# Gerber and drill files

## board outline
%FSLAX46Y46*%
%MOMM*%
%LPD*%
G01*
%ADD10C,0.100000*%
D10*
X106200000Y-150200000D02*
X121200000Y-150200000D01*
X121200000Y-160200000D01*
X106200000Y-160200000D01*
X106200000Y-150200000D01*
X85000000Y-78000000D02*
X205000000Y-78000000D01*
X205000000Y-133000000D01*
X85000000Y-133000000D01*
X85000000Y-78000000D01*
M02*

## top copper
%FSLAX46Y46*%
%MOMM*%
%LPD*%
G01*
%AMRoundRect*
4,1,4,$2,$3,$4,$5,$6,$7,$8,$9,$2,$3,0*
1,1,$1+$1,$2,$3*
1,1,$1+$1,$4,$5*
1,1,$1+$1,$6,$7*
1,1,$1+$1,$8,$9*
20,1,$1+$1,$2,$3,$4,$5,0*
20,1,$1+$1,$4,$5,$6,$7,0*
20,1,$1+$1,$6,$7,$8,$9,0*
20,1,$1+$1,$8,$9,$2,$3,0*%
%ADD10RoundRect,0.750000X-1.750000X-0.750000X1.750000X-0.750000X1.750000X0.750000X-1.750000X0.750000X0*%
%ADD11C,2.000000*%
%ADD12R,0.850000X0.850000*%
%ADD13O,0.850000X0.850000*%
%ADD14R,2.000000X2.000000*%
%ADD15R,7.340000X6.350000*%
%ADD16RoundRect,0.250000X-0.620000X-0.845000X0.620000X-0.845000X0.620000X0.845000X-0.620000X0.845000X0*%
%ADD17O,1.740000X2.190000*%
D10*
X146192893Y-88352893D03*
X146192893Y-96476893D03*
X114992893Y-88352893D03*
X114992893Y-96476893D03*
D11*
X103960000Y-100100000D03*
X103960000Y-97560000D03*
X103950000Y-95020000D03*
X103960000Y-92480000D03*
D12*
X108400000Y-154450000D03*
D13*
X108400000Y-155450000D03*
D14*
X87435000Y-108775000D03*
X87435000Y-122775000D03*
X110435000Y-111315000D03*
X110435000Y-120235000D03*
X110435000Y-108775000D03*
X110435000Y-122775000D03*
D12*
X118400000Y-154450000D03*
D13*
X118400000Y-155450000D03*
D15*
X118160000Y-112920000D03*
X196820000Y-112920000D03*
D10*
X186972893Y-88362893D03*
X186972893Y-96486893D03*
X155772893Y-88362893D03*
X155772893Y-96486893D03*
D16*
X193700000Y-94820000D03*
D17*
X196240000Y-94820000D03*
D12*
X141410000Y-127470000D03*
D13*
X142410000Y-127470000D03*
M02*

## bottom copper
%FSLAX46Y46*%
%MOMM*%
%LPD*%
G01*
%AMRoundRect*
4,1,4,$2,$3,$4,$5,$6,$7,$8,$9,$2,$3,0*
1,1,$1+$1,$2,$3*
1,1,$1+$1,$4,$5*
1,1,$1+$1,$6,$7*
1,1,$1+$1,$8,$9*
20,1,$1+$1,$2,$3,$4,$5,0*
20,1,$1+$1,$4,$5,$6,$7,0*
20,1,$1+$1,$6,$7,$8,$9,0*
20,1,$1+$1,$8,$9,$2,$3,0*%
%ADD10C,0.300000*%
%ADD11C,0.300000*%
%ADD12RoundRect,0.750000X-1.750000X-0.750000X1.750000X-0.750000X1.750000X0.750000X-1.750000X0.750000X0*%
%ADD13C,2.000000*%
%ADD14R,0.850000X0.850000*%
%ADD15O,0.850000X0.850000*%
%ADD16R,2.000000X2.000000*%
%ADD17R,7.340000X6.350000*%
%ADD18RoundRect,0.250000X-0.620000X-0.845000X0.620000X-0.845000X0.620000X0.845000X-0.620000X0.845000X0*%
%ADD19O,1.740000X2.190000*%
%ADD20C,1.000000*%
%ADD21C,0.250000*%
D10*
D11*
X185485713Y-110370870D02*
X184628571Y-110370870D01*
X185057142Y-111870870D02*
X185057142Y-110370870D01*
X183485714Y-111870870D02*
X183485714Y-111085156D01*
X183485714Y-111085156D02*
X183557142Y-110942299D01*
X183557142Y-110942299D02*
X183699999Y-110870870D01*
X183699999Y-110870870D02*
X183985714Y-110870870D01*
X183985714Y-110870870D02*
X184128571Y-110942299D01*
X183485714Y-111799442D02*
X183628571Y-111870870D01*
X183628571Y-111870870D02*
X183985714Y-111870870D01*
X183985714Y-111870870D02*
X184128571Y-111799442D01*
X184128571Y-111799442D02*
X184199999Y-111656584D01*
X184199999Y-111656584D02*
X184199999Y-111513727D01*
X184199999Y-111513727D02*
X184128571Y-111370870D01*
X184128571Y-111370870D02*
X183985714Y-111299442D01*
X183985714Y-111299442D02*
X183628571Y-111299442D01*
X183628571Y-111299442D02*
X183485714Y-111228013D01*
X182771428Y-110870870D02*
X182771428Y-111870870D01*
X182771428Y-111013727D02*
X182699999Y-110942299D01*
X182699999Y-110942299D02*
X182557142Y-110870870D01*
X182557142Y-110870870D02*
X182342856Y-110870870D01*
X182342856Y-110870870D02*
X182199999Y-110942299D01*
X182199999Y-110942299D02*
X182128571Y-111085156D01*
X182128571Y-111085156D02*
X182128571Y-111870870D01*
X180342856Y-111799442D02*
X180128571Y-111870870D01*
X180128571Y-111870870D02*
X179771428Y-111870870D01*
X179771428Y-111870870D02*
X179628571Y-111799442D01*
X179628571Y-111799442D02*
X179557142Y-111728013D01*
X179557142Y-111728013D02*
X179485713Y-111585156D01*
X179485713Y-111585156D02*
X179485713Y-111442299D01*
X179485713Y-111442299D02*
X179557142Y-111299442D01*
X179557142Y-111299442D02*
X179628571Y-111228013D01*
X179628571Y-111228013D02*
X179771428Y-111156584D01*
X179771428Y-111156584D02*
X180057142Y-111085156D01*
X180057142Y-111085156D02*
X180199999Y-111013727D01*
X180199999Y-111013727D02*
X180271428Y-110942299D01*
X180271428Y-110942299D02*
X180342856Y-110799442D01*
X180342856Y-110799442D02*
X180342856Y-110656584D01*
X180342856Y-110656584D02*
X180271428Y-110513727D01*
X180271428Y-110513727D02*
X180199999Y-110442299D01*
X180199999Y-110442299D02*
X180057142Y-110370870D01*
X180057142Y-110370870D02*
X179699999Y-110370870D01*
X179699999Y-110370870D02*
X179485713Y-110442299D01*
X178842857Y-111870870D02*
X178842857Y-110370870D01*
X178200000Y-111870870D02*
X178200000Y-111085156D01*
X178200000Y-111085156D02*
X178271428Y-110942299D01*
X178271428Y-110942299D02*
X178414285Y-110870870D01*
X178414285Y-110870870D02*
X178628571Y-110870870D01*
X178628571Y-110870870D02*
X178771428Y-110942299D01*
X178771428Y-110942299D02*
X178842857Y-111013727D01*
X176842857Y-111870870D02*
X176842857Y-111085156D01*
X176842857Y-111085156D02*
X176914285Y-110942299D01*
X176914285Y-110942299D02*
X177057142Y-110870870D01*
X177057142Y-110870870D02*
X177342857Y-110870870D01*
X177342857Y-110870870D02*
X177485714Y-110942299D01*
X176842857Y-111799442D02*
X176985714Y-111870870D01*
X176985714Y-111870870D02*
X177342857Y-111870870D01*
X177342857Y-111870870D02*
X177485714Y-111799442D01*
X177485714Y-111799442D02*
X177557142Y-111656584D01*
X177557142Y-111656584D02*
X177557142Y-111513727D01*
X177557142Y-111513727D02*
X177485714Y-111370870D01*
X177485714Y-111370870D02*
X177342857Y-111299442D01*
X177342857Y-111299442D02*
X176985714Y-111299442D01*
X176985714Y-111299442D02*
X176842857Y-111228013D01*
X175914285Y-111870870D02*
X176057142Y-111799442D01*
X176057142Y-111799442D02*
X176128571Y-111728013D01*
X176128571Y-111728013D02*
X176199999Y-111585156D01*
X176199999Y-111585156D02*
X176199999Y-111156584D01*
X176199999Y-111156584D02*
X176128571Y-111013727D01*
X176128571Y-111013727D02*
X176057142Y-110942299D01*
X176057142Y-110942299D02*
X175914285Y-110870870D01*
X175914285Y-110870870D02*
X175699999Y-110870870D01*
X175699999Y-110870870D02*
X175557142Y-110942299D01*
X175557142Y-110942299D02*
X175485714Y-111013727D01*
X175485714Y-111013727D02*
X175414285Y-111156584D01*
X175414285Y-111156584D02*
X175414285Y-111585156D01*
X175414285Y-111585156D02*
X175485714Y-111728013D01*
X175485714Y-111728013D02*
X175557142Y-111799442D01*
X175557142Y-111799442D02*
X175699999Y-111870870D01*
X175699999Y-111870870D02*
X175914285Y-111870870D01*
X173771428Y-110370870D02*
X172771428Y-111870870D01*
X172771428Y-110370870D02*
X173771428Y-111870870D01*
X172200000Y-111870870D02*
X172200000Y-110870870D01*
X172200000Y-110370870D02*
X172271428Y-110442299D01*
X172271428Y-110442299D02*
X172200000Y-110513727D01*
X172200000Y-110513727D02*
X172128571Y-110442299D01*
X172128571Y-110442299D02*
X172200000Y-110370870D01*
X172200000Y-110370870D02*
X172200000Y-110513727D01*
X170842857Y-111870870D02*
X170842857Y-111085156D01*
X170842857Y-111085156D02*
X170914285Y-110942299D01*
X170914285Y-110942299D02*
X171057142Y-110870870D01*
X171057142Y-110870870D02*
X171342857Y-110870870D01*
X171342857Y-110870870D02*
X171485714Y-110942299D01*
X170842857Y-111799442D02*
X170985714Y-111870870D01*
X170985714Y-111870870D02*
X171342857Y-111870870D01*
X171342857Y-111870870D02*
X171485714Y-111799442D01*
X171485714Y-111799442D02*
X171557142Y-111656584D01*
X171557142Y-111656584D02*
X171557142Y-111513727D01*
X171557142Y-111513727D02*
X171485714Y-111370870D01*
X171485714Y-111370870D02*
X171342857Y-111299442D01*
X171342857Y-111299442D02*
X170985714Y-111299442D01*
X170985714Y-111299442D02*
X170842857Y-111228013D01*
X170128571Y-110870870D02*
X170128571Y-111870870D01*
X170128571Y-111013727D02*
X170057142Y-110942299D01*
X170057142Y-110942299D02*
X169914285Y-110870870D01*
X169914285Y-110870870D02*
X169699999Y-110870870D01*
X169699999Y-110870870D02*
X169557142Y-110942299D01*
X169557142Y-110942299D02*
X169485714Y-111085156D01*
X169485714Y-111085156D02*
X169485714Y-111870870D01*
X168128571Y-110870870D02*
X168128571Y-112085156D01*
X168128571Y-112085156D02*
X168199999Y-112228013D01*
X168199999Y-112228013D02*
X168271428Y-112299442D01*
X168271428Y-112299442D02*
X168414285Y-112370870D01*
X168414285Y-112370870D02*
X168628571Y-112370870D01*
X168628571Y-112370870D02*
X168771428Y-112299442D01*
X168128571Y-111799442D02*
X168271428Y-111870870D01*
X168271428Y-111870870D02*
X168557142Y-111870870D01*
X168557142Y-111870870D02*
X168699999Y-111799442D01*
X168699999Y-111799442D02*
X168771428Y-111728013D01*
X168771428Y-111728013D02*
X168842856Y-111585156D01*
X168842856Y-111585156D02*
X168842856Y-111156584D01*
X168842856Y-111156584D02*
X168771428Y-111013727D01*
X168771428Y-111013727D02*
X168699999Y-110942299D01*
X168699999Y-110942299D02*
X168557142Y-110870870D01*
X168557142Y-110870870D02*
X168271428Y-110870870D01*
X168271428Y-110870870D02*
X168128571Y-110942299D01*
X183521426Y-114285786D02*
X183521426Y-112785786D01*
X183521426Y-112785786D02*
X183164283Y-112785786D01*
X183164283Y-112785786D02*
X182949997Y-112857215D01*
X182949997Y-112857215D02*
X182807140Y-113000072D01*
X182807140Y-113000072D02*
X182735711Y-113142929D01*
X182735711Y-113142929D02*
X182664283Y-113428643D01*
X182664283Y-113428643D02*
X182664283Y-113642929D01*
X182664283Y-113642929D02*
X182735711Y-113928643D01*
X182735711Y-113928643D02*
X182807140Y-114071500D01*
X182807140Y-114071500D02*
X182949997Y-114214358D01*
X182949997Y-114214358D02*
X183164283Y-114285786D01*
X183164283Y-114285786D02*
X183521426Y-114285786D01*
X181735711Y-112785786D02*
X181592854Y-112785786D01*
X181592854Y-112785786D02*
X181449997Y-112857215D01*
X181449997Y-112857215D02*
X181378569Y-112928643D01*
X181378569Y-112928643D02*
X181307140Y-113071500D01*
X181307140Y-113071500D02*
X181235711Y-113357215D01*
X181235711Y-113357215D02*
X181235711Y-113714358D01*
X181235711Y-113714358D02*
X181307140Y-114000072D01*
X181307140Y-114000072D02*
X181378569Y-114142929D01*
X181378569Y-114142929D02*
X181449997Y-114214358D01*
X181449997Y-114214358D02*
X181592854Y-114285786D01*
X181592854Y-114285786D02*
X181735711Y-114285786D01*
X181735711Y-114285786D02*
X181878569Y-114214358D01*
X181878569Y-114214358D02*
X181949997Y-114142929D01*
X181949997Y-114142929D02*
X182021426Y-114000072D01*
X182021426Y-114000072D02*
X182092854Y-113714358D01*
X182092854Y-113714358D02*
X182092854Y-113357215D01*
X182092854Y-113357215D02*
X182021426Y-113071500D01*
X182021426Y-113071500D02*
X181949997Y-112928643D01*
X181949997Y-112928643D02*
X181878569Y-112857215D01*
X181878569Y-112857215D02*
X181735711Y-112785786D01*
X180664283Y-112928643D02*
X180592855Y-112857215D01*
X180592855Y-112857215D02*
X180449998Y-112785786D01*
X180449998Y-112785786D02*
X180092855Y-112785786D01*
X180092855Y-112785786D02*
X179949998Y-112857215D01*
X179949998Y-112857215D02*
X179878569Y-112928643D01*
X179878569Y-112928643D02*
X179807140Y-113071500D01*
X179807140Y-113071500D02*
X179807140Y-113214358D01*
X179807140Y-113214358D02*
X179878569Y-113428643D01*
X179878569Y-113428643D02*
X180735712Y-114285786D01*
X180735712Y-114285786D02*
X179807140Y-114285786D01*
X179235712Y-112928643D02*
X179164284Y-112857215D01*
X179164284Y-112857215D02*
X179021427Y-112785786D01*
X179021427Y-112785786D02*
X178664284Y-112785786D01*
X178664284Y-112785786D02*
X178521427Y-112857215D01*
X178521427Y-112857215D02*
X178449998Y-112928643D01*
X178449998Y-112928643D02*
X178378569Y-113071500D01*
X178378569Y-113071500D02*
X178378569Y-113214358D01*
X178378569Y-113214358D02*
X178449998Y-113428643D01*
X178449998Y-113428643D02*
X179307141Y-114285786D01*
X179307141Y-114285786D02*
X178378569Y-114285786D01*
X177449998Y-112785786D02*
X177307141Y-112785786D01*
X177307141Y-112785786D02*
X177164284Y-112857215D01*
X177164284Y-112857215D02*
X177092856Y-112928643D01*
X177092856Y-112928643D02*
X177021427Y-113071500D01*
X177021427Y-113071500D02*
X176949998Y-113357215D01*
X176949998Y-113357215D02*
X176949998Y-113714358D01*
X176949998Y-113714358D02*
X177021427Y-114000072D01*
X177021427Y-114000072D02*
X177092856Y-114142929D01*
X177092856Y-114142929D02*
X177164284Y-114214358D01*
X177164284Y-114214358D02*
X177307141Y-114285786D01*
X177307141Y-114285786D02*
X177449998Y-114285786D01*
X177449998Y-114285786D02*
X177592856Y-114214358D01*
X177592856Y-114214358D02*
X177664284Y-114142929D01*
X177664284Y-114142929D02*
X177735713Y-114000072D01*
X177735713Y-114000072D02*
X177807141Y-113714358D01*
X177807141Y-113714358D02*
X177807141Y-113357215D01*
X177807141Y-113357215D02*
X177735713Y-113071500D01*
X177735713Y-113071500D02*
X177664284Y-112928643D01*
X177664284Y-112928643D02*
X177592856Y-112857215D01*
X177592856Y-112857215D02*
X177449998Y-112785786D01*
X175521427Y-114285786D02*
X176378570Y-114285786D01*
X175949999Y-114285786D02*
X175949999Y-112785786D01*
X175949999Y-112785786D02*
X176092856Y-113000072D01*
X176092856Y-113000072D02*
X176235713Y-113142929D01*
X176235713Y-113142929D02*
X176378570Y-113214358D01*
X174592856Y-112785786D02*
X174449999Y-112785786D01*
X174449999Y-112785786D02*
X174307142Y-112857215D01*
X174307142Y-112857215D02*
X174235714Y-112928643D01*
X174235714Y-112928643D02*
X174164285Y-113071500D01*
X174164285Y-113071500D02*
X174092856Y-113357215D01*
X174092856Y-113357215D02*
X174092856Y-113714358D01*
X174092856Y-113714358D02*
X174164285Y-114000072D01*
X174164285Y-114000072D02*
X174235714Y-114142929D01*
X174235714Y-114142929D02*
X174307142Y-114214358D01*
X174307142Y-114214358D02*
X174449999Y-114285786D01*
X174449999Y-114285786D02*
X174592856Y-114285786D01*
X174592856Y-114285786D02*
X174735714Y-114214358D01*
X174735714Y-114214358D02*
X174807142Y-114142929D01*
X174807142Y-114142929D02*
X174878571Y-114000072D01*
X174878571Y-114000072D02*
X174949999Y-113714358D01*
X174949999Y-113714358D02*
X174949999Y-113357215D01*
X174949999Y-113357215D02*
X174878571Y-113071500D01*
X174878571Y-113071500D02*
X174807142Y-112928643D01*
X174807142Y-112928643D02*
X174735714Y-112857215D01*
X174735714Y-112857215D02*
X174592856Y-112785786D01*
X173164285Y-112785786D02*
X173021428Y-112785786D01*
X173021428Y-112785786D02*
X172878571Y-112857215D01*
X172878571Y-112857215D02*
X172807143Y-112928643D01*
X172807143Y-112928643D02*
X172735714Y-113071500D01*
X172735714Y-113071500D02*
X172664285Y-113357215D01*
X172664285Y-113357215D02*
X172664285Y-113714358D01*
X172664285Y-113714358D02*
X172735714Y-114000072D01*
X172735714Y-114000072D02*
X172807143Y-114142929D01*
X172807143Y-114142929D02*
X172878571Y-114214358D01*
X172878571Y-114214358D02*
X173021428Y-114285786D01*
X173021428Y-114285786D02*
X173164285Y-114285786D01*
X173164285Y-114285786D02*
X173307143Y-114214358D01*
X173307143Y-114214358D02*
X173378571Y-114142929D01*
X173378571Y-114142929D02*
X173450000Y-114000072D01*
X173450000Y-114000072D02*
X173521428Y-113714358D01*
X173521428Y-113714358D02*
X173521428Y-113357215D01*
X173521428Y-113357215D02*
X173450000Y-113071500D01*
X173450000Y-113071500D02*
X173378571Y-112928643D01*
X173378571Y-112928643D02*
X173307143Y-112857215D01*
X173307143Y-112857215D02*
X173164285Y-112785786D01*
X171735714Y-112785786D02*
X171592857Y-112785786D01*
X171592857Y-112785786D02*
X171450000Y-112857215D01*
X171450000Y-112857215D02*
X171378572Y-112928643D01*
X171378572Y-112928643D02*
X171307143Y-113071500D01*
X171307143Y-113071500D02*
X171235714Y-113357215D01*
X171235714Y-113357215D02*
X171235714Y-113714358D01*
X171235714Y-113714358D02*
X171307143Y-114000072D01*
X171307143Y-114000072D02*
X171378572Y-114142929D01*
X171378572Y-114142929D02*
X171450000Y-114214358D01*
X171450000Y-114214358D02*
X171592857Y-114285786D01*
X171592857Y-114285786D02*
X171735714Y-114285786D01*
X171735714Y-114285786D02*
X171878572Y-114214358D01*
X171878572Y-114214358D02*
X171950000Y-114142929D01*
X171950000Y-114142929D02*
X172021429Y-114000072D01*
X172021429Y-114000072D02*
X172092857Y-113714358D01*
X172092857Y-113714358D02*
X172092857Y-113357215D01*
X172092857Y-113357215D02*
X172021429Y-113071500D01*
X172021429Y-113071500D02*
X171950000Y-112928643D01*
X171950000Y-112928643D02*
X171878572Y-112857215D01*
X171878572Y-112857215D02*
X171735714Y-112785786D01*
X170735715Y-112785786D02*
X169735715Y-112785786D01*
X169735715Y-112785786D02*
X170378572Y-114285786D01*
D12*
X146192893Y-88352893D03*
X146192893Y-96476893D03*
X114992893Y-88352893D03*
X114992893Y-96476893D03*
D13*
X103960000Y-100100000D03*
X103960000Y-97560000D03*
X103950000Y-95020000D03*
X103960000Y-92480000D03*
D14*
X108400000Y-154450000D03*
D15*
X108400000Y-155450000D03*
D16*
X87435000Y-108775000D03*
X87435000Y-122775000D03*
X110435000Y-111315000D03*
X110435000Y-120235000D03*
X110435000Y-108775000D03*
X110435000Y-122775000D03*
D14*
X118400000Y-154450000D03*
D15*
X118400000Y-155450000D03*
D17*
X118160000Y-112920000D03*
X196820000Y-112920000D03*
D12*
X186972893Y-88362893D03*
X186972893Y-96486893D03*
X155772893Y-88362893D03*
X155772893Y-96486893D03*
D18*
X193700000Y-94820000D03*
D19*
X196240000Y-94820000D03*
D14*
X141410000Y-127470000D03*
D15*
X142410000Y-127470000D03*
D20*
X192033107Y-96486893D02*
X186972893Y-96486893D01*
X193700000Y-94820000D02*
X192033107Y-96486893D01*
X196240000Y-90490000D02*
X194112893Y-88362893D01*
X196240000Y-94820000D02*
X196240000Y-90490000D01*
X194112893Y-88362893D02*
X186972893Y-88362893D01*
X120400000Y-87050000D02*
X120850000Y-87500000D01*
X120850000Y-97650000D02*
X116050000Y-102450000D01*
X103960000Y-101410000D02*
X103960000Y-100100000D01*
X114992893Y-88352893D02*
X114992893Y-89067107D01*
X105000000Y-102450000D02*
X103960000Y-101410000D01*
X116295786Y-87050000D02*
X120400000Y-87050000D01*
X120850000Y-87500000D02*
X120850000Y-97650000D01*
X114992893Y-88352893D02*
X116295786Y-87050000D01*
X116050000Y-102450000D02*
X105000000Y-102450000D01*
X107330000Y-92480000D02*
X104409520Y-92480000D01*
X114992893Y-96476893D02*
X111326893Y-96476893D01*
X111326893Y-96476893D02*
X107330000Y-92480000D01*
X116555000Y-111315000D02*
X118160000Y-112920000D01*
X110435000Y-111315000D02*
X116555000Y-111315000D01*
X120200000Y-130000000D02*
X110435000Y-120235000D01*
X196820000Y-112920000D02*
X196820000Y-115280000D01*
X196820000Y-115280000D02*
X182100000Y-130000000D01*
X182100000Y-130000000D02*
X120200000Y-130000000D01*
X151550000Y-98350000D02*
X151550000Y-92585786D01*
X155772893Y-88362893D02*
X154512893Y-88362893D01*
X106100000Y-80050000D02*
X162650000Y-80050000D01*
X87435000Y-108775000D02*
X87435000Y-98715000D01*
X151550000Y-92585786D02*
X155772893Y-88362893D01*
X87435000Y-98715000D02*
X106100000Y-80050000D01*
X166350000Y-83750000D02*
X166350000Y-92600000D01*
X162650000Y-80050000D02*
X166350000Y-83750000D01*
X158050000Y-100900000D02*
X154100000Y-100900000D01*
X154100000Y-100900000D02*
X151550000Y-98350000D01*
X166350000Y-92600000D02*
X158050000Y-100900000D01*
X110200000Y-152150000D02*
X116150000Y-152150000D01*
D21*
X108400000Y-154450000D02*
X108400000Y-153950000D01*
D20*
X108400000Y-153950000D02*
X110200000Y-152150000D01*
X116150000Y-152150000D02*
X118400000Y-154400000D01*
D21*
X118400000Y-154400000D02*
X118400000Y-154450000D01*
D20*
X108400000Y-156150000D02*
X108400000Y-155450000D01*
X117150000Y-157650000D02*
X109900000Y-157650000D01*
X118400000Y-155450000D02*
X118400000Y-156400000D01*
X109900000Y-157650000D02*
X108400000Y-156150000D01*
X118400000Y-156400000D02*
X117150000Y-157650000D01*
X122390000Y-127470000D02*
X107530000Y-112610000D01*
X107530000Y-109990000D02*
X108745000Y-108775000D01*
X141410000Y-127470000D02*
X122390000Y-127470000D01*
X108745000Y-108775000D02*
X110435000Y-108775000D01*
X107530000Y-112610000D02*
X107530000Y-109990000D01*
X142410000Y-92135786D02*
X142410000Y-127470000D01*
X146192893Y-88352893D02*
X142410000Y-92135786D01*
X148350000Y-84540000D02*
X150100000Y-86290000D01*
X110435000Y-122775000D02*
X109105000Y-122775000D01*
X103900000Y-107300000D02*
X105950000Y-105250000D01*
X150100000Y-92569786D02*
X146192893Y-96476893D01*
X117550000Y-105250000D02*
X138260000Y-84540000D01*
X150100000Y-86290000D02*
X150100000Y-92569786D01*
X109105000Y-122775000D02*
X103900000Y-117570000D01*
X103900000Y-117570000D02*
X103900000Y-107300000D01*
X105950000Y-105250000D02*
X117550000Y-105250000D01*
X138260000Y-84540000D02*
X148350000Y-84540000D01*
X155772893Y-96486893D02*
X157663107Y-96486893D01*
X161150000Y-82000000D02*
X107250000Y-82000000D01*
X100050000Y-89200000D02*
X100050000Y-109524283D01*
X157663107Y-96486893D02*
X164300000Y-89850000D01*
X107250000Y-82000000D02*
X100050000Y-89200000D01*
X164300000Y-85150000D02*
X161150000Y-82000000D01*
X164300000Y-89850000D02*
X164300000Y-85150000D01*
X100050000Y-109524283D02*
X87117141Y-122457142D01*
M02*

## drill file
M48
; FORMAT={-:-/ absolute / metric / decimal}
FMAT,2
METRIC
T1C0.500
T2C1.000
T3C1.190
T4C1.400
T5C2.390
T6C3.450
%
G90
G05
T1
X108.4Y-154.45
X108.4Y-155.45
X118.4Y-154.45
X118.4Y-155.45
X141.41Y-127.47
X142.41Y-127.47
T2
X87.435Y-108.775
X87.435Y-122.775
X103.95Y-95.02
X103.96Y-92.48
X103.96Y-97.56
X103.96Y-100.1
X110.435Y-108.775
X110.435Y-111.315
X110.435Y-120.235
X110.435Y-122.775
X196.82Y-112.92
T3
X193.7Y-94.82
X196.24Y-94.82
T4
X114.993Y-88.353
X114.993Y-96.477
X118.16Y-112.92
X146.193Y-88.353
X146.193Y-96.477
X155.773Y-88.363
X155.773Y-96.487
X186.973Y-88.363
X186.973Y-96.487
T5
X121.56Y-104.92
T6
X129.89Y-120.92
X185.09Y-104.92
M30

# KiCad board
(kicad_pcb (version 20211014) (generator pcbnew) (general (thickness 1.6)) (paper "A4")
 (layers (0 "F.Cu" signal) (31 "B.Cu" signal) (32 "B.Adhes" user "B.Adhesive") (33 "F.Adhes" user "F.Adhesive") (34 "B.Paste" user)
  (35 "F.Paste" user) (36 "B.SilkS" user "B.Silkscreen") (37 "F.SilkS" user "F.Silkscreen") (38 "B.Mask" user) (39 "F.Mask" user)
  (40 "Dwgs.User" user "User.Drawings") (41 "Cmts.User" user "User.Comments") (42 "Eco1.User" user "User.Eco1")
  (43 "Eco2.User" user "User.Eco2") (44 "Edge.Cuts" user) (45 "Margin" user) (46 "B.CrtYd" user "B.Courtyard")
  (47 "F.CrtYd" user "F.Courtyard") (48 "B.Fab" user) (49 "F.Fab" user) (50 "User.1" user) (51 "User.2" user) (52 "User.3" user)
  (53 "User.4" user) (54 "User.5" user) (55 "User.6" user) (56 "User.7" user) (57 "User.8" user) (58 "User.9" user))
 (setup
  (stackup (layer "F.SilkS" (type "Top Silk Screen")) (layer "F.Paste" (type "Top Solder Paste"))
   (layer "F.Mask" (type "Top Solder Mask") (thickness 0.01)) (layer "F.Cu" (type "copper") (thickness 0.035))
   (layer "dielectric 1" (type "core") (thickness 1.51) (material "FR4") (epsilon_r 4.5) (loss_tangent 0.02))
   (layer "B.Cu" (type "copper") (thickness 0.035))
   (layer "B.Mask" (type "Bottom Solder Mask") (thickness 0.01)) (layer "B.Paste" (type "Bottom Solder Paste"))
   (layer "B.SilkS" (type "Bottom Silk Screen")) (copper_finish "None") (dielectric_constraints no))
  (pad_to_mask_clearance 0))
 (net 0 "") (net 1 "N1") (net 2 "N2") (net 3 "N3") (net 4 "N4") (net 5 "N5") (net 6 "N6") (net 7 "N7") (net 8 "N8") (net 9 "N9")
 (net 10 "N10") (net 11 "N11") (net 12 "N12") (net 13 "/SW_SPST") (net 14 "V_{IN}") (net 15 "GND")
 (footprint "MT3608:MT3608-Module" (layer "F.Cu") (at 112.092893 83.852893)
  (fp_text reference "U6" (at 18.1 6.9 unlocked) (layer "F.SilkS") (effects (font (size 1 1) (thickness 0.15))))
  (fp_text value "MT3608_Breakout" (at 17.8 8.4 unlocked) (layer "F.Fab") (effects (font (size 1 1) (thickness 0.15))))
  (pad "1" thru_hole roundrect (at 34.1 4.5) (size 5 3) (drill 1.4) (layers *.Cu *.Mask) (roundrect_rratio 0.25) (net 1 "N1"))
  (pad "2" thru_hole roundrect (at 34.1 12.624) (size 5 3) (drill 1.4) (layers *.Cu *.Mask) (roundrect_rratio 0.25) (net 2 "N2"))
  (pad "3" thru_hole roundrect (at 2.9 4.5) (size 5 3) (drill 1.4) (layers *.Cu *.Mask) (roundrect_rratio 0.25) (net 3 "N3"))
  (pad "4" thru_hole roundrect (at 2.9 12.624) (size 5 3) (drill 1.4) (layers *.Cu *.Mask) (roundrect_rratio 0.25) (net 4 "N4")))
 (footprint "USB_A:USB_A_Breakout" (layer "F.Cu") (at 84.98 104.79)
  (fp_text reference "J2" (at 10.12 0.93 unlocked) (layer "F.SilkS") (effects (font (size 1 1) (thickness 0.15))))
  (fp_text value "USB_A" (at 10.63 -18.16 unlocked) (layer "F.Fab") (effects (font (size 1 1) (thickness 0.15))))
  (pad "1" thru_hole circle (at 18.98 -4.69 180) (size 2 2) (drill 1) (layers *.Cu *.Mask) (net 3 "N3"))
  (pad "2" thru_hole circle (at 18.98 -7.23 180) (size 2 2) (drill 1) (layers *.Cu *.Mask) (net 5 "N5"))
  (pad "3" thru_hole circle (at 18.97 -9.77 180) (size 2 2) (drill 1) (layers *.Cu *.Mask) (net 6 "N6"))
  (pad "4" thru_hole circle (at 18.98 -12.31 180) (size 2 2) (drill 1) (layers *.Cu *.Mask) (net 4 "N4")))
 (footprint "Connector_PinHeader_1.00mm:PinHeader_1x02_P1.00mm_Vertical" (layer "F.Cu") (at 108.4 154.45)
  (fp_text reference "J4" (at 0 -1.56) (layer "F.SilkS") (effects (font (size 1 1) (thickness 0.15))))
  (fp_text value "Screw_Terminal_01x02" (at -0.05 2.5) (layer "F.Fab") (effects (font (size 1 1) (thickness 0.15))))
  (pad "1" thru_hole rect (at 0 0) (size 0.85 0.85) (drill 0.5) (layers *.Cu *.Mask) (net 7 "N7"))
  (pad "2" thru_hole oval (at 0 1) (size 0.85 0.85) (drill 0.5) (layers *.Cu *.Mask) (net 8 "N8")))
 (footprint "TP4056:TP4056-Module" (layer "F.Cu") (at 84.935 124.375)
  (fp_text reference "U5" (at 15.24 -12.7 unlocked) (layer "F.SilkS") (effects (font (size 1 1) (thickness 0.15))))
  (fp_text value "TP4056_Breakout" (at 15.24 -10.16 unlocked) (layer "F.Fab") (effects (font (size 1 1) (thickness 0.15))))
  (pad "1" thru_hole rect (at 2.5 -15.6) (size 2 2) (drill 1) (layers *.Cu *.Mask) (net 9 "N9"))
  (pad "2" thru_hole rect (at 2.5 -1.6) (size 2 2) (drill 1) (layers *.Cu *.Mask) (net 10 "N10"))
  (pad "3" thru_hole rect (at 25.5 -13.06) (size 2 2) (drill 1) (layers *.Cu *.Mask) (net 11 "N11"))
  (pad "4" thru_hole rect (at 25.5 -4.14) (size 2 2) (drill 1) (layers *.Cu *.Mask) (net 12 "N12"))
  (pad "5" thru_hole rect (at 25.5 -15.6 90) (size 2 2) (drill 1) (layers *.Cu *.Mask) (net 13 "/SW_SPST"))
  (pad "6" thru_hole rect (at 25.5 -1.6) (size 2 2) (drill 1) (layers *.Cu *.Mask) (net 2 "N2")))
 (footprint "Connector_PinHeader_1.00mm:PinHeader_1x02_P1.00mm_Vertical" (layer "F.Cu") (at 118.4 154.45)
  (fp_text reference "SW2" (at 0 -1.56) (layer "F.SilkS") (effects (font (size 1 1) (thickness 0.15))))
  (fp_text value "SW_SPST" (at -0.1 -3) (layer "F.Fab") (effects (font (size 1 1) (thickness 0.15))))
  (pad "1" thru_hole rect (at 0 0) (size 0.85 0.85) (drill 0.5) (layers *.Cu *.Mask) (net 7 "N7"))
  (pad "2" thru_hole oval (at 0 1) (size 0.85 0.85) (drill 0.5) (layers *.Cu *.Mask) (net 8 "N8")))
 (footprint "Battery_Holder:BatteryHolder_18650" (layer "F.Cu") (at 157.49 112.92)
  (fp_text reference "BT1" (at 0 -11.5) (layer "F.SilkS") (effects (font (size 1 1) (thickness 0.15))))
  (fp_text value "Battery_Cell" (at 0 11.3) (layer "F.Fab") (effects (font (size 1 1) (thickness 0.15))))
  (pad "" np_thru_hole circle (at -35.93 -8) (size 2.39 2.39) (drill 2.39) (layers *.Cu *.Mask))
  (pad "" np_thru_hole circle (at 27.6 -8) (size 3.45 3.45) (drill 3.45) (layers *.Cu *.Mask))
  (pad "" np_thru_hole circle (at -27.6 8) (size 3.45 3.45) (drill 3.45) (layers *.Cu *.Mask))
  (pad "1" thru_hole rect (at -39.33 0) (size 7.34 6.35) (drill 1.4) (layers *.Cu *.Mask) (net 11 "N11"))
  (pad "2" thru_hole rect (at 39.33 0) (size 7.34 6.35) (drill 1) (layers *.Cu *.Mask) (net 12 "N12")))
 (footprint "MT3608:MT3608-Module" (layer "F.Cu") (at 152.872893 83.862893)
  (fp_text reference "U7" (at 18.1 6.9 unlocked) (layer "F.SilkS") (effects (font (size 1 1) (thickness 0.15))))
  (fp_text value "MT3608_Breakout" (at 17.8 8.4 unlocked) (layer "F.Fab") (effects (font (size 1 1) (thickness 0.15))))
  (pad "1" thru_hole roundrect (at 34.1 4.5) (size 5 3) (drill 1.4) (layers *.Cu *.Mask) (roundrect_rratio 0.25) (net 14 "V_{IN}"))
  (pad "2" thru_hole roundrect (at 34.1 12.624) (size 5 3) (drill 1.4) (layers *.Cu *.Mask) (roundrect_rratio 0.25) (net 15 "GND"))
  (pad "3" thru_hole roundrect (at 2.9 4.5) (size 5 3) (drill 1.4) (layers *.Cu *.Mask) (roundrect_rratio 0.25) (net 9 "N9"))
  (pad "4" thru_hole roundrect (at 2.9 12.624) (size 5 3) (drill 1.4) (layers *.Cu *.Mask) (roundrect_rratio 0.25) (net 10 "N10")))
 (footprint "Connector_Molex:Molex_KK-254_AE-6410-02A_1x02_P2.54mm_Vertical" (layer "F.Cu") (at 193.7 94.82)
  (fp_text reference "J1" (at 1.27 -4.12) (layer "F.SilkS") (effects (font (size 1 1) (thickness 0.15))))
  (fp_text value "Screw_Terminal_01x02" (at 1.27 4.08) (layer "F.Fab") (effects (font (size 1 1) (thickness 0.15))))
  (pad "1" thru_hole roundrect (at 0 0) (size 1.74 2.19) (drill 1.19) (layers *.Cu *.Mask) (roundrect_rratio 0.1436781609) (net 15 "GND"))
  (pad "2" thru_hole oval (at 2.54 0) (size 1.74 2.19) (drill 1.19) (layers *.Cu *.Mask) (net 14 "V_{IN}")))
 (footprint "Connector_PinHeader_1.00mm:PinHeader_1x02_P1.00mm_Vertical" (layer "F.Cu") (at 141.41 127.47 90)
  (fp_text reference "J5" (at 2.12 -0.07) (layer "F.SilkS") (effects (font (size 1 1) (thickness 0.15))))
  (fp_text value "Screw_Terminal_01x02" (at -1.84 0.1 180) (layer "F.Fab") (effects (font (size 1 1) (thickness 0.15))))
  (pad "1" thru_hole rect (at 0 0 90) (size 0.85 0.85) (drill 0.5) (layers *.Cu *.Mask) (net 13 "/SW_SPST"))
  (pad "2" thru_hole oval (at 0 1 90) (size 0.85 0.85) (drill 0.5) (layers *.Cu *.Mask) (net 1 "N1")))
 (gr_rect (start 106.2 150.2) (end 121.2 160.2) (layer "Edge.Cuts") (width 0.1) (fill none))
 (gr_rect (start 85 78) (end 205 133) (layer "Edge.Cuts") (width 0.1) (fill none))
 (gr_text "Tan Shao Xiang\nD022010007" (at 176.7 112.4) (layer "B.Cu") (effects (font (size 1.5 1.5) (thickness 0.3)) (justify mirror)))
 (segment (start 192.033107 96.486893) (end 186.972893 96.486893) (width 1) (layer "B.Cu") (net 15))
 (segment (start 193.7 94.82) (end 192.033107 96.486893) (width 1) (layer "B.Cu") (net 15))
 (segment (start 196.24 90.49) (end 194.112893 88.362893) (width 1) (layer "B.Cu") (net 14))
 (segment (start 196.24 94.82) (end 196.24 90.49) (width 1) (layer "B.Cu") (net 14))
 (segment (start 194.112893 88.362893) (end 186.972893 88.362893) (width 1) (layer "B.Cu") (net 14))
 (segment (start 120.4 87.05) (end 120.85 87.5) (width 1) (layer "B.Cu") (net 3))
 (segment (start 120.85 97.65) (end 116.05 102.45) (width 1) (layer "B.Cu") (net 3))
 (segment (start 103.96 101.41) (end 103.96 100.1) (width 1) (layer "B.Cu") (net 3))
 (segment (start 114.992893 88.352893) (end 114.992893 89.067107) (width 1) (layer "B.Cu") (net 3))
 (segment (start 105 102.45) (end 103.96 101.41) (width 1) (layer "B.Cu") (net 3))
 (segment (start 116.295786 87.05) (end 120.4 87.05) (width 1) (layer "B.Cu") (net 3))
 (segment (start 120.85 87.5) (end 120.85 97.65) (width 1) (layer "B.Cu") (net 3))
 (segment (start 114.992893 88.352893) (end 116.295786 87.05) (width 1) (layer "B.Cu") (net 3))
 (segment (start 116.05 102.45) (end 105 102.45) (width 1) (layer "B.Cu") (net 3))
 (segment (start 107.33 92.48) (end 104.40952 92.48) (width 1) (layer "B.Cu") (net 4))
 (segment (start 114.992893 96.476893) (end 111.326893 96.476893) (width 1) (layer "B.Cu") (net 4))
 (segment (start 111.326893 96.476893) (end 107.33 92.48) (width 1) (layer "B.Cu") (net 4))
 (segment (start 116.555 111.315) (end 118.16 112.92) (width 1) (layer "B.Cu") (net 11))
 (segment (start 110.435 111.315) (end 116.555 111.315) (width 1) (layer "B.Cu") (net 11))
 (segment (start 120.2 130) (end 110.435 120.235) (width 1) (layer "B.Cu") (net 12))
 (segment (start 196.82 112.92) (end 196.82 115.28) (width 1) (layer "B.Cu") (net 12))
 (segment (start 196.82 115.28) (end 182.1 130) (width 1) (layer "B.Cu") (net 12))
 (segment (start 182.1 130) (end 120.2 130) (width 1) (layer "B.Cu") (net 12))
 (segment (start 151.55 98.35) (end 151.55 92.585786) (width 1) (layer "B.Cu") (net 9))
 (segment (start 155.772893 88.362893) (end 154.512893 88.362893) (width 1) (layer "B.Cu") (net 9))
 (segment (start 106.1 80.05) (end 162.65 80.05) (width 1) (layer "B.Cu") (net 9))
 (segment (start 87.435 108.775) (end 87.435 98.715) (width 1) (layer "B.Cu") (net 9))
 (segment (start 151.55 92.585786) (end 155.772893 88.362893) (width 1) (layer "B.Cu") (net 9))
 (segment (start 87.435 98.715) (end 106.1 80.05) (width 1) (layer "B.Cu") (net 9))
 (segment (start 166.35 83.75) (end 166.35 92.6) (width 1) (layer "B.Cu") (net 9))
 (segment (start 162.65 80.05) (end 166.35 83.75) (width 1) (layer "B.Cu") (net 9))
 (segment (start 158.05 100.9) (end 154.1 100.9) (width 1) (layer "B.Cu") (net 9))
 (segment (start 154.1 100.9) (end 151.55 98.35) (width 1) (layer "B.Cu") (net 9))
 (segment (start 166.35 92.6) (end 158.05 100.9) (width 1) (layer "B.Cu") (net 9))
 (segment (start 110.2 152.15) (end 116.15 152.15) (width 1) (layer "B.Cu") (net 7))
 (segment (start 108.4 154.45) (end 108.4 153.95) (width 0.25) (layer "B.Cu") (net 7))
 (segment (start 108.4 153.95) (end 110.2 152.15) (width 1) (layer "B.Cu") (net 7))
 (segment (start 116.15 152.15) (end 118.4 154.4) (width 1) (layer "B.Cu") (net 7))
 (segment (start 118.4 154.4) (end 118.4 154.45) (width 0.25) (layer "B.Cu") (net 7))
 (segment (start 108.4 156.15) (end 108.4 155.45) (width 1) (layer "B.Cu") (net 8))
 (segment (start 117.15 157.65) (end 109.9 157.65) (width 1) (layer "B.Cu") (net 8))
 (segment (start 118.4 155.45) (end 118.4 156.4) (width 1) (layer "B.Cu") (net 8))
 (segment (start 109.9 157.65) (end 108.4 156.15) (width 1) (layer "B.Cu") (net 8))
 (segment (start 118.4 156.4) (end 117.15 157.65) (width 1) (layer "B.Cu") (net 8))
 (segment (start 122.39 127.47) (end 107.53 112.61) (width 1) (layer "B.Cu") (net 13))
 (segment (start 107.53 109.99) (end 108.745 108.775) (width 1) (layer "B.Cu") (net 13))
 (segment (start 141.41 127.47) (end 122.39 127.47) (width 1) (layer "B.Cu") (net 13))
 (segment (start 108.745 108.775) (end 110.435 108.775) (width 1) (layer "B.Cu") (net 13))
 (segment (start 107.53 112.61) (end 107.53 109.99) (width 1) (layer "B.Cu") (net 13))
 (segment (start 142.41 92.135786) (end 142.41 127.47) (width 1) (layer "B.Cu") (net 1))
 (segment (start 146.192893 88.352893) (end 142.41 92.135786) (width 1) (layer "B.Cu") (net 1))
 (segment (start 148.35 84.54) (end 150.1 86.29) (width 1) (layer "B.Cu") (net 2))
 (segment (start 110.435 122.775) (end 109.105 122.775) (width 1) (layer "B.Cu") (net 2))
 (segment (start 103.9 107.3) (end 105.95 105.25) (width 1) (layer "B.Cu") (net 2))
 (segment (start 150.1 92.569786) (end 146.192893 96.476893) (width 1) (layer "B.Cu") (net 2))
 (segment (start 117.55 105.25) (end 138.26 84.54) (width 1) (layer "B.Cu") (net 2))
 (segment (start 150.1 86.29) (end 150.1 92.569786) (width 1) (layer "B.Cu") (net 2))
 (segment (start 109.105 122.775) (end 103.9 117.57) (width 1) (layer "B.Cu") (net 2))
 (segment (start 103.9 117.57) (end 103.9 107.3) (width 1) (layer "B.Cu") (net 2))
 (segment (start 105.95 105.25) (end 117.55 105.25) (width 1) (layer "B.Cu") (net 2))
 (segment (start 138.26 84.54) (end 148.35 84.54) (width 1) (layer "B.Cu") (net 2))
 (segment (start 155.772893 96.486893) (end 157.663107 96.486893) (width 1) (layer "B.Cu") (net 10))
 (segment (start 161.15 82) (end 107.25 82) (width 1) (layer "B.Cu") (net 10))
 (segment (start 100.05 89.2) (end 100.05 109.524283) (width 1) (layer "B.Cu") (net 10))
 (segment (start 157.663107 96.486893) (end 164.3 89.85) (width 1) (layer "B.Cu") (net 10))
 (segment (start 107.25 82) (end 100.05 89.2) (width 1) (layer "B.Cu") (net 10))
 (segment (start 164.3 85.15) (end 161.15 82) (width 1) (layer "B.Cu") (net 10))
 (segment (start 164.3 89.85) (end 164.3 85.15) (width 1) (layer "B.Cu") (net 10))
 (segment (start 100.05 109.524283) (end 87.117141 122.457142) (width 1) (layer "B.Cu") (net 10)))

